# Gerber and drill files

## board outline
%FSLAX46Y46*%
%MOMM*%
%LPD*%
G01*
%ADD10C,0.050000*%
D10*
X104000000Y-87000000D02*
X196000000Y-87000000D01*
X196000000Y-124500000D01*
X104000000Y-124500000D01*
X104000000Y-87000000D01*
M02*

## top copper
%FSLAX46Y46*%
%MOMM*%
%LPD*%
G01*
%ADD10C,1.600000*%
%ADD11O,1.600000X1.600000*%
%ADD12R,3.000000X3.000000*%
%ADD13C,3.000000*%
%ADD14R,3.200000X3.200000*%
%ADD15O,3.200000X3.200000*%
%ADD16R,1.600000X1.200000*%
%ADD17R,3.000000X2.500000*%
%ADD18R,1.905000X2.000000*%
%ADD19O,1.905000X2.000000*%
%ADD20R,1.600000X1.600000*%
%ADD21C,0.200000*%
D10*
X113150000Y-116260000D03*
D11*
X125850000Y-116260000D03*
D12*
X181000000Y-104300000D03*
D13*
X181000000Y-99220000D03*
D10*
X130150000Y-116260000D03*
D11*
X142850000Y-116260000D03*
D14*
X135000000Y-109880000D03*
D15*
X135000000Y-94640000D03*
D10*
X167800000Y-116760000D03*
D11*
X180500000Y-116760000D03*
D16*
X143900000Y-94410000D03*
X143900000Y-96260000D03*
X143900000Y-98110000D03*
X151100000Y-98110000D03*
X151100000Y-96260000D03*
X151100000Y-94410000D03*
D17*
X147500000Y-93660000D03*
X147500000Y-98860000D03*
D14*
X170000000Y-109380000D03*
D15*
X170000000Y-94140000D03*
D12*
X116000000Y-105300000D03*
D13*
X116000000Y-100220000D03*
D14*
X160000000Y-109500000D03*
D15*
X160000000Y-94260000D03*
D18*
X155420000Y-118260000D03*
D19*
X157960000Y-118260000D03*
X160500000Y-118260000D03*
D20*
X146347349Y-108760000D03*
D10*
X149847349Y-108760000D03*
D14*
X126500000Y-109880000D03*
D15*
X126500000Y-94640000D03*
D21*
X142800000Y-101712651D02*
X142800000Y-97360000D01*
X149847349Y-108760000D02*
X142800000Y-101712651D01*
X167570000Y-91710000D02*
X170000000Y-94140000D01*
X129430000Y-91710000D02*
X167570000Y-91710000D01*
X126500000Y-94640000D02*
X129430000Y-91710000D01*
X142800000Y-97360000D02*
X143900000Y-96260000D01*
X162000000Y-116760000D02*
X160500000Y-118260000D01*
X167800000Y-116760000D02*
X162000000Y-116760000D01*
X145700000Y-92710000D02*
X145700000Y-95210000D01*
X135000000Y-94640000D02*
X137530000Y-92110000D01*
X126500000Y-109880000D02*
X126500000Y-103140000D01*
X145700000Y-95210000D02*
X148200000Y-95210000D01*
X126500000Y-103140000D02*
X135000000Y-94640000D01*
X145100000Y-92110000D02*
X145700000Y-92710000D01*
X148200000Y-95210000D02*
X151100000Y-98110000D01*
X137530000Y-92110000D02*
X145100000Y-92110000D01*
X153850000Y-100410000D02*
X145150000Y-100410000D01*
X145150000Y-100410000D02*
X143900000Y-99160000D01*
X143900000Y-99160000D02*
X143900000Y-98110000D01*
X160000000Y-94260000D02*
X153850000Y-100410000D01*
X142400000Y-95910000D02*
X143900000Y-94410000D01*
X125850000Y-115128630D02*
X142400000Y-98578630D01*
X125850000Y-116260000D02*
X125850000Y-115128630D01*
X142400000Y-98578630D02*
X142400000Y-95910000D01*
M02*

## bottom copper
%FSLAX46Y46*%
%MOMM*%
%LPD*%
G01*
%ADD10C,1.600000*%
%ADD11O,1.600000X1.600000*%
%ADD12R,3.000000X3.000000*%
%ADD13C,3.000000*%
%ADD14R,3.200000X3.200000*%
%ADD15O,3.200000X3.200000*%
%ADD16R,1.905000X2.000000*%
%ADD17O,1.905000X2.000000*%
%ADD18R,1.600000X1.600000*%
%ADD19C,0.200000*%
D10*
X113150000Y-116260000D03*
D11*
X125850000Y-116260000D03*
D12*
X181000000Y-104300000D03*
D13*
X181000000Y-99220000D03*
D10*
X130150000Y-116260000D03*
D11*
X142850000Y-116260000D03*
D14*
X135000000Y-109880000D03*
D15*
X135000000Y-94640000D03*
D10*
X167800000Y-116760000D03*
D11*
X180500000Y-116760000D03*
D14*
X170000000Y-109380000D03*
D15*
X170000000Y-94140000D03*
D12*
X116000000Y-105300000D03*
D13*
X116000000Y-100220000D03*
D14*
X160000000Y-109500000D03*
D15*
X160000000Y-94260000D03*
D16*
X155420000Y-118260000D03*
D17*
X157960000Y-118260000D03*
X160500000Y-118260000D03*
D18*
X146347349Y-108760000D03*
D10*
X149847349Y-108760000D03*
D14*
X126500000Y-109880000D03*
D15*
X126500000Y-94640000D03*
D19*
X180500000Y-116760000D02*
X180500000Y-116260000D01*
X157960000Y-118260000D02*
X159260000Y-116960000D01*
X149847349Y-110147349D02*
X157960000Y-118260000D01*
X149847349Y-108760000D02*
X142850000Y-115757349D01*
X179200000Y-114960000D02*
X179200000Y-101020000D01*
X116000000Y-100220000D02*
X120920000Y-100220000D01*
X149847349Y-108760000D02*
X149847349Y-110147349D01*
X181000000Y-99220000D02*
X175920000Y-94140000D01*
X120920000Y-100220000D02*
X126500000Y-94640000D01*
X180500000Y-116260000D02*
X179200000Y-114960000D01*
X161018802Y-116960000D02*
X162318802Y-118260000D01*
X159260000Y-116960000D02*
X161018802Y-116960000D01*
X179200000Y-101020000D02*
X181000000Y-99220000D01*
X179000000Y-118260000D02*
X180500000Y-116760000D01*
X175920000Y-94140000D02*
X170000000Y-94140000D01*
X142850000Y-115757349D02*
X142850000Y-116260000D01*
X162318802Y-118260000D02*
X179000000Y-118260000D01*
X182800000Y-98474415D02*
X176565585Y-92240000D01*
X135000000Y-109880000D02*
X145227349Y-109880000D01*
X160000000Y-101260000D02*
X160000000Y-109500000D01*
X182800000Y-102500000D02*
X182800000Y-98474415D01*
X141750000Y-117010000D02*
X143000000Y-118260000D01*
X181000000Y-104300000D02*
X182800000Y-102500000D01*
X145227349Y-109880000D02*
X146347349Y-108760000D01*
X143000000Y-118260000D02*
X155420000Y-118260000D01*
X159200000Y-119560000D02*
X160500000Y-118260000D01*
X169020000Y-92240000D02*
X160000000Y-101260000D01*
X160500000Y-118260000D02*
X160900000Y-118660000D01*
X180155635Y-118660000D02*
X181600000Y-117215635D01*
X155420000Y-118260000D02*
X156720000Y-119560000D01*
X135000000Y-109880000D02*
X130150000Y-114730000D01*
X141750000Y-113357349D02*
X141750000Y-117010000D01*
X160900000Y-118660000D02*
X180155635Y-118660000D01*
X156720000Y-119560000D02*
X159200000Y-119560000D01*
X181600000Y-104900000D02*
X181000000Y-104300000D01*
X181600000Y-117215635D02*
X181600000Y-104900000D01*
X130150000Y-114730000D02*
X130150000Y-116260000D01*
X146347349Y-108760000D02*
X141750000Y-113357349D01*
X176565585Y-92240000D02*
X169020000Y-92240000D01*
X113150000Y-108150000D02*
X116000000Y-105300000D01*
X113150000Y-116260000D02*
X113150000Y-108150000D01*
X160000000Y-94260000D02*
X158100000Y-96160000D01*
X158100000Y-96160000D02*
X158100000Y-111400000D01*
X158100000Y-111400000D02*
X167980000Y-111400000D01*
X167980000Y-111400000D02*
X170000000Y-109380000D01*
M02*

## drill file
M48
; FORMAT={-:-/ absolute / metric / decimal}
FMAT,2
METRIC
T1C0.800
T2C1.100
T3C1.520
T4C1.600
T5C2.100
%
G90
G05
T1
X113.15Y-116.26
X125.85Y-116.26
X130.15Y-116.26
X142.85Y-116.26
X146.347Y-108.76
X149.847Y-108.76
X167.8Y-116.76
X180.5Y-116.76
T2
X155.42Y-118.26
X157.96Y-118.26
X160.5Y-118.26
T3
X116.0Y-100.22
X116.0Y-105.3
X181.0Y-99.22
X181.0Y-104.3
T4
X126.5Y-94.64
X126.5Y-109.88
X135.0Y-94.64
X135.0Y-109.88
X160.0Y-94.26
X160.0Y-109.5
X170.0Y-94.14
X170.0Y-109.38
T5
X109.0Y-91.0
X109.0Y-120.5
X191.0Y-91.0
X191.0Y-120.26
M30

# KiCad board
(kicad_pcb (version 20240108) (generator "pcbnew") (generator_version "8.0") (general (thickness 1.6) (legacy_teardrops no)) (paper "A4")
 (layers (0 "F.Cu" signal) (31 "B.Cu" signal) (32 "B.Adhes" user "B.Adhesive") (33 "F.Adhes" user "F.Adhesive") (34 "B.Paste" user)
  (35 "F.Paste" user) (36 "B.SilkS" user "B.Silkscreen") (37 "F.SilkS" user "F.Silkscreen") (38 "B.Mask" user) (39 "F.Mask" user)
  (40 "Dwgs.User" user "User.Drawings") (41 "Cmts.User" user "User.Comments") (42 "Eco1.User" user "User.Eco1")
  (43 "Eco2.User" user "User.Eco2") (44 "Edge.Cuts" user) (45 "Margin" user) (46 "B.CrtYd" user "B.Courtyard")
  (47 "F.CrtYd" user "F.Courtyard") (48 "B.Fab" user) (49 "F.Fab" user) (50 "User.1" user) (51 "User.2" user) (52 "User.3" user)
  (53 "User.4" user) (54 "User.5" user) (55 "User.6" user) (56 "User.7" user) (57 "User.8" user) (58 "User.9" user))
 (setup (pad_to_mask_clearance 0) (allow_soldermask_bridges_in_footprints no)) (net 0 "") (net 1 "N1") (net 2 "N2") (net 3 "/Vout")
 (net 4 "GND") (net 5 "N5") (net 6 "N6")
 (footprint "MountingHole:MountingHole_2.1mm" (layer "F.Cu") (at 109 91)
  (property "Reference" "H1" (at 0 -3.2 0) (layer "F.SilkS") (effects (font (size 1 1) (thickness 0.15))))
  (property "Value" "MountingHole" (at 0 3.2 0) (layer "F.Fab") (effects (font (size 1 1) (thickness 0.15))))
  (pad "" np_thru_hole circle (at 0 0) (size 2.1 2.1) (drill 2.1) (layers "*.Cu" "*.Mask")))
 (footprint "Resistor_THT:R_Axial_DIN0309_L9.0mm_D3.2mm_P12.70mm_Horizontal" (layer "F.Cu") (at 113.15 116.26)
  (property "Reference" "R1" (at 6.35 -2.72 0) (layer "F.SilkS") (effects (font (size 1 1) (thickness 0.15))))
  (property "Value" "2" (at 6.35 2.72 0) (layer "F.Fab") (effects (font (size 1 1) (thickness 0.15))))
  (pad "1" thru_hole circle (at 0 0) (size 1.6 1.6) (drill 0.8) (layers "*.Cu" "*.Mask") (remove_unused_layers no) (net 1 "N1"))
  (pad "2" thru_hole oval (at 12.7 0) (size 1.6 1.6) (drill 0.8) (layers "*.Cu" "*.Mask") (remove_unused_layers no) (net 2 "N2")))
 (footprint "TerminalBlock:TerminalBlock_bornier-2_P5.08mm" (layer "F.Cu") (at 181 104.3 90)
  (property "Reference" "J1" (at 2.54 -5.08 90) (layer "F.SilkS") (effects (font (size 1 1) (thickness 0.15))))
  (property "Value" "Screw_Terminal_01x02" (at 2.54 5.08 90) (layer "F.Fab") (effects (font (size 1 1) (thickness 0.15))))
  (pad "1" thru_hole rect (at 0 0 90) (size 3 3) (drill 1.52) (layers "*.Cu" "*.Mask") (remove_unused_layers no) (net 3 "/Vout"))
  (pad "2" thru_hole circle (at 5.08 0 90) (size 3 3) (drill 1.52) (layers "*.Cu" "*.Mask") (remove_unused_layers no) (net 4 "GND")))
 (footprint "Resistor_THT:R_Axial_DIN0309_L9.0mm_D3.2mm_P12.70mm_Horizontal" (layer "F.Cu") (at 130.15 116.26)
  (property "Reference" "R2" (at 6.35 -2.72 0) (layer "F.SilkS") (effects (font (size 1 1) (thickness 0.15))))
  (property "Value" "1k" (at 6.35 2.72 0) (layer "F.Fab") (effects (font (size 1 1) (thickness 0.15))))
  (pad "1" thru_hole circle (at 0 0) (size 1.6 1.6) (drill 0.8) (layers "*.Cu" "*.Mask") (remove_unused_layers no) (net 3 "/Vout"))
  (pad "2" thru_hole oval (at 12.7 0) (size 1.6 1.6) (drill 0.8) (layers "*.Cu" "*.Mask") (remove_unused_layers no) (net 4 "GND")))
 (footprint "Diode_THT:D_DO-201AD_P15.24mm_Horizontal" (layer "F.Cu") (at 135 109.88 90)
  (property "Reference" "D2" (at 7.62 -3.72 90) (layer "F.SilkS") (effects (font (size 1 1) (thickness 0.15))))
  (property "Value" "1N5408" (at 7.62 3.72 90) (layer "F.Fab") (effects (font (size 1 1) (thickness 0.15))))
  (pad "1" thru_hole rect (at 0 0 90) (size 3.2 3.2) (drill 1.6) (layers "*.Cu" "*.Mask") (remove_unused_layers no) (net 3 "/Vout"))
  (pad "2" thru_hole oval (at 15.24 0 90) (size 3.2 3.2) (drill 1.6) (layers "*.Cu" "*.Mask") (remove_unused_layers no) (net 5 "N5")))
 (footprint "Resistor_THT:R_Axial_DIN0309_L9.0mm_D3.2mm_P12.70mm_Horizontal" (layer "F.Cu") (at 167.8 116.76)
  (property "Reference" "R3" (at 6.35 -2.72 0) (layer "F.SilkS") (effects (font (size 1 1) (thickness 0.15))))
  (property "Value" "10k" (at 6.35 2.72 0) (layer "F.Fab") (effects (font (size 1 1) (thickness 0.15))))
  (pad "1" thru_hole circle (at 0 0) (size 1.6 1.6) (drill 0.8) (layers "*.Cu" "*.Mask") (remove_unused_layers no) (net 3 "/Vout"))
  (pad "2" thru_hole oval (at 12.7 0) (size 1.6 1.6) (drill 0.8) (layers "*.Cu" "*.Mask") (remove_unused_layers no) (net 4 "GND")))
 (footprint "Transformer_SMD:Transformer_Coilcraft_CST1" (layer "F.Cu") (at 147.5 96.26)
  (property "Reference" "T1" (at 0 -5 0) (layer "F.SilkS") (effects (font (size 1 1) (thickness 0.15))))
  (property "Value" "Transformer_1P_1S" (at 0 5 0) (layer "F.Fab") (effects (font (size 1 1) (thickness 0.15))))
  (pad "1" smd rect (at -3.6 -1.85) (size 1.6 1.2) (layers "F.Cu" "F.Paste" "F.Mask") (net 2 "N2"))
  (pad "2" smd rect (at -3.6 0) (size 1.6 1.2) (layers "F.Cu" "F.Paste" "F.Mask") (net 4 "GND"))
  (pad "3" smd rect (at -3.6 1.85) (size 1.6 1.2) (layers "F.Cu" "F.Paste" "F.Mask") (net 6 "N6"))
  (pad "4" smd rect (at 3.6 1.85) (size 1.6 1.2) (layers "F.Cu" "F.Paste" "F.Mask") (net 5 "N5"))
  (pad "5" smd rect (at 3.6 0) (size 1.6 1.2) (layers "F.Cu" "F.Paste" "F.Mask"))
  (pad "6" smd rect (at 3.6 -1.85) (size 1.6 1.2) (layers "F.Cu" "F.Paste" "F.Mask"))
  (pad "7" smd rect (at 0 -2.6) (size 3 2.5) (layers "F.Cu" "F.Paste" "F.Mask"))
  (pad "8" smd rect (at 0 2.6) (size 3 2.5) (layers "F.Cu" "F.Paste" "F.Mask")))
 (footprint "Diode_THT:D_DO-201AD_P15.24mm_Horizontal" (layer "F.Cu") (at 170 109.38 90)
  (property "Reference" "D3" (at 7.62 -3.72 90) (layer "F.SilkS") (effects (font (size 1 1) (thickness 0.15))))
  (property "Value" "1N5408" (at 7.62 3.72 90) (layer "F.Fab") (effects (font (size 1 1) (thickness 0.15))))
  (pad "1" thru_hole rect (at 0 0 90) (size 3.2 3.2) (drill 1.6) (layers "*.Cu" "*.Mask") (remove_unused_layers no) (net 6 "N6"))
  (pad "2" thru_hole oval (at 15.24 0 90) (size 3.2 3.2) (drill 1.6) (layers "*.Cu" "*.Mask") (remove_unused_layers no) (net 4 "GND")))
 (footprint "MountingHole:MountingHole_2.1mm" (layer "F.Cu") (at 191 120.26)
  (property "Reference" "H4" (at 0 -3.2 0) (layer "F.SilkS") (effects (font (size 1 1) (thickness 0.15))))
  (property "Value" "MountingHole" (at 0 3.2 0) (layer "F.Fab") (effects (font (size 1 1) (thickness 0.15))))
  (pad "" np_thru_hole circle (at 0 0) (size 2.1 2.1) (drill 2.1) (layers "*.Cu" "*.Mask")))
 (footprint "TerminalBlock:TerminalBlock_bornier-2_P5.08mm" (layer "F.Cu") (at 116 105.3 90)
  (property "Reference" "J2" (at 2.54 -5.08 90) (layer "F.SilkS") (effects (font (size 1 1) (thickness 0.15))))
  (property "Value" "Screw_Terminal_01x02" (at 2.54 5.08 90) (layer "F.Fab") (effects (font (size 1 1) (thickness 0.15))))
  (pad "1" thru_hole rect (at 0 0 90) (size 3 3) (drill 1.52) (layers "*.Cu" "*.Mask") (remove_unused_layers no) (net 1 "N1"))
  (pad "2" thru_hole circle (at 5.08 0 90) (size 3 3) (drill 1.52) (layers "*.Cu" "*.Mask") (remove_unused_layers no) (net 4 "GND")))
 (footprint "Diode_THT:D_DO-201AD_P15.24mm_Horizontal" (layer "F.Cu") (at 160 109.5 90)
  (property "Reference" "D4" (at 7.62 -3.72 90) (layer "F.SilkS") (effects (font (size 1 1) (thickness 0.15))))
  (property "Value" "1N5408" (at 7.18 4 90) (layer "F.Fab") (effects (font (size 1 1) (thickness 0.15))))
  (pad "1" thru_hole rect (at 0 0 90) (size 3.2 3.2) (drill 1.6) (layers "*.Cu" "*.Mask") (remove_unused_layers no) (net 3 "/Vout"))
  (pad "2" thru_hole oval (at 15.24 0 90) (size 3.2 3.2) (drill 1.6) (layers "*.Cu" "*.Mask") (remove_unused_layers no) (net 6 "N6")))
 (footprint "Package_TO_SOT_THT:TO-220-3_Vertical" (layer "F.Cu") (at 155.42 118.26)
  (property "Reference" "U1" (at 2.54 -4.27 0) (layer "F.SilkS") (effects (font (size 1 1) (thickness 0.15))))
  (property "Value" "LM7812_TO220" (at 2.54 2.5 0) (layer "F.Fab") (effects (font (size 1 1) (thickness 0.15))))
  (pad "1" thru_hole rect (at 0 0) (size 1.905 2) (drill 1.1) (layers "*.Cu" "*.Mask") (remove_unused_layers no) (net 3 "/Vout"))
  (pad "2" thru_hole oval (at 2.54 0) (size 1.905 2) (drill 1.1) (layers "*.Cu" "*.Mask") (remove_unused_layers no) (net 4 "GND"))
  (pad "3" thru_hole oval (at 5.08 0) (size 1.905 2) (drill 1.1) (layers "*.Cu" "*.Mask") (remove_unused_layers no) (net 3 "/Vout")))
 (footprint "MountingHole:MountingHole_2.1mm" (layer "F.Cu") (at 109 120.5)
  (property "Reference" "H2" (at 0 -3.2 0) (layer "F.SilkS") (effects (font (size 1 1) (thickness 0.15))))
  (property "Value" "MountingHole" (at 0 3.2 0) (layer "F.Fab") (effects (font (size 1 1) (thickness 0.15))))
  (pad "" np_thru_hole circle (at 0 0) (size 2.1 2.1) (drill 2.1) (layers "*.Cu" "*.Mask")))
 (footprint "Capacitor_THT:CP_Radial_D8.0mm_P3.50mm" (layer "F.Cu") (at 146.347349 108.76)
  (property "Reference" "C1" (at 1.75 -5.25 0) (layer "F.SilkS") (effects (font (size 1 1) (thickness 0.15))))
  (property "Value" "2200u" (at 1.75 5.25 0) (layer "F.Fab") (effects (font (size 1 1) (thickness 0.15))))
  (pad "1" thru_hole rect (at 0 0) (size 1.6 1.6) (drill 0.8) (layers "*.Cu" "*.Mask") (remove_unused_layers no) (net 3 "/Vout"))
  (pad "2" thru_hole circle (at 3.5 0) (size 1.6 1.6) (drill 0.8) (layers "*.Cu" "*.Mask") (remove_unused_layers no) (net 4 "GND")))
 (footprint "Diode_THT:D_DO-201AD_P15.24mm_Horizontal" (layer "F.Cu") (at 126.5 109.88 90)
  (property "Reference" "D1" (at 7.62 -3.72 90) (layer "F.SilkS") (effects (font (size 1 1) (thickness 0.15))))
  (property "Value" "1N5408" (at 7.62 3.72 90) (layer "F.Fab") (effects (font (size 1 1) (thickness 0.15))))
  (pad "1" thru_hole rect (at 0 0 90) (size 3.2 3.2) (drill 1.6) (layers "*.Cu" "*.Mask") (remove_unused_layers no) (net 5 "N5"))
  (pad "2" thru_hole oval (at 15.24 0 90) (size 3.2 3.2) (drill 1.6) (layers "*.Cu" "*.Mask") (remove_unused_layers no) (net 4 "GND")))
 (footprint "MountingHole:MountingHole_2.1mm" (layer "F.Cu") (at 191 91)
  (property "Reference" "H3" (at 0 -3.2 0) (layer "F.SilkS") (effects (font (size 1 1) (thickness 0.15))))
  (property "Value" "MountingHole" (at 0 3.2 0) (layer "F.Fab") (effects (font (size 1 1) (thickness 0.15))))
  (pad "" np_thru_hole circle (at 0 0) (size 2.1 2.1) (drill 2.1) (layers "*.Cu" "*.Mask")))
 (gr_rect (start 104 87) (end 196 124.5) (stroke (width 0.05) (type default)) (fill none) (layer "Edge.Cuts"))
 (segment (start 142.8 101.712651) (end 142.8 97.36) (width 0.2) (layer "F.Cu") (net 4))
 (segment (start 149.847349 108.76) (end 142.8 101.712651) (width 0.2) (layer "F.Cu") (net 4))
 (segment (start 167.57 91.71) (end 170 94.14) (width 0.2) (layer "F.Cu") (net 4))
 (segment (start 129.43 91.71) (end 167.57 91.71) (width 0.2) (layer "F.Cu") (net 4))
 (segment (start 126.5 94.64) (end 129.43 91.71) (width 0.2) (layer "F.Cu") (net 4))
 (segment (start 142.8 97.36) (end 143.9 96.26) (width 0.2) (layer "F.Cu") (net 4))
 (segment (start 180.5 116.76) (end 180.5 116.26) (width 0.2) (layer "B.Cu") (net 4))
 (segment (start 157.96 118.26) (end 159.26 116.96) (width 0.2) (layer "B.Cu") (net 4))
 (segment (start 149.847349 110.147349) (end 157.96 118.26) (width 0.2) (layer "B.Cu") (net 4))
 (segment (start 149.847349 108.76) (end 142.85 115.757349) (width 0.2) (layer "B.Cu") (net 4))
 (segment (start 179.2 114.96) (end 179.2 101.02) (width 0.2) (layer "B.Cu") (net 4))
 (segment (start 116 100.22) (end 120.92 100.22) (width 0.2) (layer "B.Cu") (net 4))
 (segment (start 149.847349 108.76) (end 149.847349 110.147349) (width 0.2) (layer "B.Cu") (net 4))
 (segment (start 181 99.22) (end 175.92 94.14) (width 0.2) (layer "B.Cu") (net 4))
 (segment (start 120.92 100.22) (end 126.5 94.64) (width 0.2) (layer "B.Cu") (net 4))
 (segment (start 180.5 116.26) (end 179.2 114.96) (width 0.2) (layer "B.Cu") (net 4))
 (segment (start 161.018802 116.96) (end 162.318802 118.26) (width 0.2) (layer "B.Cu") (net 4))
 (segment (start 159.26 116.96) (end 161.018802 116.96) (width 0.2) (layer "B.Cu") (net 4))
 (segment (start 179.2 101.02) (end 181 99.22) (width 0.2) (layer "B.Cu") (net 4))
 (segment (start 179 118.26) (end 180.5 116.76) (width 0.2) (layer "B.Cu") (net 4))
 (segment (start 175.92 94.14) (end 170 94.14) (width 0.2) (layer "B.Cu") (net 4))
 (segment (start 142.85 115.757349) (end 142.85 116.26) (width 0.2) (layer "B.Cu") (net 4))
 (segment (start 162.318802 118.26) (end 179 118.26) (width 0.2) (layer "B.Cu") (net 4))
 (segment (start 162 116.76) (end 160.5 118.26) (width 0.2) (layer "F.Cu") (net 3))
 (segment (start 167.8 116.76) (end 162 116.76) (width 0.2) (layer "F.Cu") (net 3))
 (segment (start 182.8 98.474415) (end 176.565585 92.24) (width 0.2) (layer "B.Cu") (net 3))
 (segment (start 135 109.88) (end 145.227349 109.88) (width 0.2) (layer "B.Cu") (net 3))
 (segment (start 160 101.26) (end 160 109.5) (width 0.2) (layer "B.Cu") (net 3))
 (segment (start 182.8 102.5) (end 182.8 98.474415) (width 0.2) (layer "B.Cu") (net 3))
 (segment (start 141.75 117.01) (end 143 118.26) (width 0.2) (layer "B.Cu") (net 3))
 (segment (start 181 104.3) (end 182.8 102.5) (width 0.2) (layer "B.Cu") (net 3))
 (segment (start 145.227349 109.88) (end 146.347349 108.76) (width 0.2) (layer "B.Cu") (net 3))
 (segment (start 143 118.26) (end 155.42 118.26) (width 0.2) (layer "B.Cu") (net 3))
 (segment (start 159.2 119.56) (end 160.5 118.26) (width 0.2) (layer "B.Cu") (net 3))
 (segment (start 169.02 92.24) (end 160 101.26) (width 0.2) (layer "B.Cu") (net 3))
 (segment (start 160.5 118.26) (end 160.9 118.66) (width 0.2) (layer "B.Cu") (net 3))
 (segment (start 180.155635 118.66) (end 181.6 117.215635) (width 0.2) (layer "B.Cu") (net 3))
 (segment (start 155.42 118.26) (end 156.72 119.56) (width 0.2) (layer "B.Cu") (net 3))
 (segment (start 135 109.88) (end 130.15 114.73) (width 0.2) (layer "B.Cu") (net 3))
 (segment (start 141.75 113.357349) (end 141.75 117.01) (width 0.2) (layer "B.Cu") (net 3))
 (segment (start 160.9 118.66) (end 180.155635 118.66) (width 0.2) (layer "B.Cu") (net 3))
 (segment (start 156.72 119.56) (end 159.2 119.56) (width 0.2) (layer "B.Cu") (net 3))
 (segment (start 181.6 104.9) (end 181 104.3) (width 0.2) (layer "B.Cu") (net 3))
 (segment (start 181.6 117.215635) (end 181.6 104.9) (width 0.2) (layer "B.Cu") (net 3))
 (segment (start 130.15 114.73) (end 130.15 116.26) (width 0.2) (layer "B.Cu") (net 3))
 (segment (start 146.347349 108.76) (end 141.75 113.357349) (width 0.2) (layer "B.Cu") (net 3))
 (segment (start 176.565585 92.24) (end 169.02 92.24) (width 0.2) (layer "B.Cu") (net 3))
 (segment (start 145.7 92.71) (end 145.7 95.21) (width 0.2) (layer "F.Cu") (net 5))
 (segment (start 135 94.64) (end 137.53 92.11) (width 0.2) (layer "F.Cu") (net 5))
 (segment (start 126.5 109.88) (end 126.5 103.14) (width 0.2) (layer "F.Cu") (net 5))
 (segment (start 145.7 95.21) (end 148.2 95.21) (width 0.2) (layer "F.Cu") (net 5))
 (segment (start 126.5 103.14) (end 135 94.64) (width 0.2) (layer "F.Cu") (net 5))
 (segment (start 145.1 92.11) (end 145.7 92.71) (width 0.2) (layer "F.Cu") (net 5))
 (segment (start 148.2 95.21) (end 151.1 98.11) (width 0.2) (layer "F.Cu") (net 5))
 (segment (start 137.53 92.11) (end 145.1 92.11) (width 0.2) (layer "F.Cu") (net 5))
 (segment (start 113.15 108.15) (end 116 105.3) (width 0.2) (layer "B.Cu") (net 1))
 (segment (start 113.15 116.26) (end 113.15 108.15) (width 0.2) (layer "B.Cu") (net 1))
 (segment (start 153.85 100.41) (end 145.15 100.41) (width 0.2) (layer "F.Cu") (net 6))
 (segment (start 145.15 100.41) (end 143.9 99.16) (width 0.2) (layer "F.Cu") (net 6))
 (segment (start 143.9 99.16) (end 143.9 98.11) (width 0.2) (layer "F.Cu") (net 6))
 (segment (start 160 94.26) (end 153.85 100.41) (width 0.2) (layer "F.Cu") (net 6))
 (segment (start 160 94.26) (end 158.1 96.16) (width 0.2) (layer "B.Cu") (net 6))
 (segment (start 158.1 96.16) (end 158.1 111.4) (width 0.2) (layer "B.Cu") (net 6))
 (segment (start 158.1 111.4) (end 167.98 111.4) (width 0.2) (layer "B.Cu") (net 6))
 (segment (start 167.98 111.4) (end 170 109.38) (width 0.2) (layer "B.Cu") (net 6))
 (segment (start 142.4 95.91) (end 143.9 94.41) (width 0.2) (layer "F.Cu") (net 2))
 (segment (start 125.85 115.12863) (end 142.4 98.57863) (width 0.2) (layer "F.Cu") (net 2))
 (segment (start 125.85 116.26) (end 125.85 115.12863) (width 0.2) (layer "F.Cu") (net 2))
 (segment (start 142.4 98.57863) (end 142.4 95.91) (width 0.2) (layer "F.Cu") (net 2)))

